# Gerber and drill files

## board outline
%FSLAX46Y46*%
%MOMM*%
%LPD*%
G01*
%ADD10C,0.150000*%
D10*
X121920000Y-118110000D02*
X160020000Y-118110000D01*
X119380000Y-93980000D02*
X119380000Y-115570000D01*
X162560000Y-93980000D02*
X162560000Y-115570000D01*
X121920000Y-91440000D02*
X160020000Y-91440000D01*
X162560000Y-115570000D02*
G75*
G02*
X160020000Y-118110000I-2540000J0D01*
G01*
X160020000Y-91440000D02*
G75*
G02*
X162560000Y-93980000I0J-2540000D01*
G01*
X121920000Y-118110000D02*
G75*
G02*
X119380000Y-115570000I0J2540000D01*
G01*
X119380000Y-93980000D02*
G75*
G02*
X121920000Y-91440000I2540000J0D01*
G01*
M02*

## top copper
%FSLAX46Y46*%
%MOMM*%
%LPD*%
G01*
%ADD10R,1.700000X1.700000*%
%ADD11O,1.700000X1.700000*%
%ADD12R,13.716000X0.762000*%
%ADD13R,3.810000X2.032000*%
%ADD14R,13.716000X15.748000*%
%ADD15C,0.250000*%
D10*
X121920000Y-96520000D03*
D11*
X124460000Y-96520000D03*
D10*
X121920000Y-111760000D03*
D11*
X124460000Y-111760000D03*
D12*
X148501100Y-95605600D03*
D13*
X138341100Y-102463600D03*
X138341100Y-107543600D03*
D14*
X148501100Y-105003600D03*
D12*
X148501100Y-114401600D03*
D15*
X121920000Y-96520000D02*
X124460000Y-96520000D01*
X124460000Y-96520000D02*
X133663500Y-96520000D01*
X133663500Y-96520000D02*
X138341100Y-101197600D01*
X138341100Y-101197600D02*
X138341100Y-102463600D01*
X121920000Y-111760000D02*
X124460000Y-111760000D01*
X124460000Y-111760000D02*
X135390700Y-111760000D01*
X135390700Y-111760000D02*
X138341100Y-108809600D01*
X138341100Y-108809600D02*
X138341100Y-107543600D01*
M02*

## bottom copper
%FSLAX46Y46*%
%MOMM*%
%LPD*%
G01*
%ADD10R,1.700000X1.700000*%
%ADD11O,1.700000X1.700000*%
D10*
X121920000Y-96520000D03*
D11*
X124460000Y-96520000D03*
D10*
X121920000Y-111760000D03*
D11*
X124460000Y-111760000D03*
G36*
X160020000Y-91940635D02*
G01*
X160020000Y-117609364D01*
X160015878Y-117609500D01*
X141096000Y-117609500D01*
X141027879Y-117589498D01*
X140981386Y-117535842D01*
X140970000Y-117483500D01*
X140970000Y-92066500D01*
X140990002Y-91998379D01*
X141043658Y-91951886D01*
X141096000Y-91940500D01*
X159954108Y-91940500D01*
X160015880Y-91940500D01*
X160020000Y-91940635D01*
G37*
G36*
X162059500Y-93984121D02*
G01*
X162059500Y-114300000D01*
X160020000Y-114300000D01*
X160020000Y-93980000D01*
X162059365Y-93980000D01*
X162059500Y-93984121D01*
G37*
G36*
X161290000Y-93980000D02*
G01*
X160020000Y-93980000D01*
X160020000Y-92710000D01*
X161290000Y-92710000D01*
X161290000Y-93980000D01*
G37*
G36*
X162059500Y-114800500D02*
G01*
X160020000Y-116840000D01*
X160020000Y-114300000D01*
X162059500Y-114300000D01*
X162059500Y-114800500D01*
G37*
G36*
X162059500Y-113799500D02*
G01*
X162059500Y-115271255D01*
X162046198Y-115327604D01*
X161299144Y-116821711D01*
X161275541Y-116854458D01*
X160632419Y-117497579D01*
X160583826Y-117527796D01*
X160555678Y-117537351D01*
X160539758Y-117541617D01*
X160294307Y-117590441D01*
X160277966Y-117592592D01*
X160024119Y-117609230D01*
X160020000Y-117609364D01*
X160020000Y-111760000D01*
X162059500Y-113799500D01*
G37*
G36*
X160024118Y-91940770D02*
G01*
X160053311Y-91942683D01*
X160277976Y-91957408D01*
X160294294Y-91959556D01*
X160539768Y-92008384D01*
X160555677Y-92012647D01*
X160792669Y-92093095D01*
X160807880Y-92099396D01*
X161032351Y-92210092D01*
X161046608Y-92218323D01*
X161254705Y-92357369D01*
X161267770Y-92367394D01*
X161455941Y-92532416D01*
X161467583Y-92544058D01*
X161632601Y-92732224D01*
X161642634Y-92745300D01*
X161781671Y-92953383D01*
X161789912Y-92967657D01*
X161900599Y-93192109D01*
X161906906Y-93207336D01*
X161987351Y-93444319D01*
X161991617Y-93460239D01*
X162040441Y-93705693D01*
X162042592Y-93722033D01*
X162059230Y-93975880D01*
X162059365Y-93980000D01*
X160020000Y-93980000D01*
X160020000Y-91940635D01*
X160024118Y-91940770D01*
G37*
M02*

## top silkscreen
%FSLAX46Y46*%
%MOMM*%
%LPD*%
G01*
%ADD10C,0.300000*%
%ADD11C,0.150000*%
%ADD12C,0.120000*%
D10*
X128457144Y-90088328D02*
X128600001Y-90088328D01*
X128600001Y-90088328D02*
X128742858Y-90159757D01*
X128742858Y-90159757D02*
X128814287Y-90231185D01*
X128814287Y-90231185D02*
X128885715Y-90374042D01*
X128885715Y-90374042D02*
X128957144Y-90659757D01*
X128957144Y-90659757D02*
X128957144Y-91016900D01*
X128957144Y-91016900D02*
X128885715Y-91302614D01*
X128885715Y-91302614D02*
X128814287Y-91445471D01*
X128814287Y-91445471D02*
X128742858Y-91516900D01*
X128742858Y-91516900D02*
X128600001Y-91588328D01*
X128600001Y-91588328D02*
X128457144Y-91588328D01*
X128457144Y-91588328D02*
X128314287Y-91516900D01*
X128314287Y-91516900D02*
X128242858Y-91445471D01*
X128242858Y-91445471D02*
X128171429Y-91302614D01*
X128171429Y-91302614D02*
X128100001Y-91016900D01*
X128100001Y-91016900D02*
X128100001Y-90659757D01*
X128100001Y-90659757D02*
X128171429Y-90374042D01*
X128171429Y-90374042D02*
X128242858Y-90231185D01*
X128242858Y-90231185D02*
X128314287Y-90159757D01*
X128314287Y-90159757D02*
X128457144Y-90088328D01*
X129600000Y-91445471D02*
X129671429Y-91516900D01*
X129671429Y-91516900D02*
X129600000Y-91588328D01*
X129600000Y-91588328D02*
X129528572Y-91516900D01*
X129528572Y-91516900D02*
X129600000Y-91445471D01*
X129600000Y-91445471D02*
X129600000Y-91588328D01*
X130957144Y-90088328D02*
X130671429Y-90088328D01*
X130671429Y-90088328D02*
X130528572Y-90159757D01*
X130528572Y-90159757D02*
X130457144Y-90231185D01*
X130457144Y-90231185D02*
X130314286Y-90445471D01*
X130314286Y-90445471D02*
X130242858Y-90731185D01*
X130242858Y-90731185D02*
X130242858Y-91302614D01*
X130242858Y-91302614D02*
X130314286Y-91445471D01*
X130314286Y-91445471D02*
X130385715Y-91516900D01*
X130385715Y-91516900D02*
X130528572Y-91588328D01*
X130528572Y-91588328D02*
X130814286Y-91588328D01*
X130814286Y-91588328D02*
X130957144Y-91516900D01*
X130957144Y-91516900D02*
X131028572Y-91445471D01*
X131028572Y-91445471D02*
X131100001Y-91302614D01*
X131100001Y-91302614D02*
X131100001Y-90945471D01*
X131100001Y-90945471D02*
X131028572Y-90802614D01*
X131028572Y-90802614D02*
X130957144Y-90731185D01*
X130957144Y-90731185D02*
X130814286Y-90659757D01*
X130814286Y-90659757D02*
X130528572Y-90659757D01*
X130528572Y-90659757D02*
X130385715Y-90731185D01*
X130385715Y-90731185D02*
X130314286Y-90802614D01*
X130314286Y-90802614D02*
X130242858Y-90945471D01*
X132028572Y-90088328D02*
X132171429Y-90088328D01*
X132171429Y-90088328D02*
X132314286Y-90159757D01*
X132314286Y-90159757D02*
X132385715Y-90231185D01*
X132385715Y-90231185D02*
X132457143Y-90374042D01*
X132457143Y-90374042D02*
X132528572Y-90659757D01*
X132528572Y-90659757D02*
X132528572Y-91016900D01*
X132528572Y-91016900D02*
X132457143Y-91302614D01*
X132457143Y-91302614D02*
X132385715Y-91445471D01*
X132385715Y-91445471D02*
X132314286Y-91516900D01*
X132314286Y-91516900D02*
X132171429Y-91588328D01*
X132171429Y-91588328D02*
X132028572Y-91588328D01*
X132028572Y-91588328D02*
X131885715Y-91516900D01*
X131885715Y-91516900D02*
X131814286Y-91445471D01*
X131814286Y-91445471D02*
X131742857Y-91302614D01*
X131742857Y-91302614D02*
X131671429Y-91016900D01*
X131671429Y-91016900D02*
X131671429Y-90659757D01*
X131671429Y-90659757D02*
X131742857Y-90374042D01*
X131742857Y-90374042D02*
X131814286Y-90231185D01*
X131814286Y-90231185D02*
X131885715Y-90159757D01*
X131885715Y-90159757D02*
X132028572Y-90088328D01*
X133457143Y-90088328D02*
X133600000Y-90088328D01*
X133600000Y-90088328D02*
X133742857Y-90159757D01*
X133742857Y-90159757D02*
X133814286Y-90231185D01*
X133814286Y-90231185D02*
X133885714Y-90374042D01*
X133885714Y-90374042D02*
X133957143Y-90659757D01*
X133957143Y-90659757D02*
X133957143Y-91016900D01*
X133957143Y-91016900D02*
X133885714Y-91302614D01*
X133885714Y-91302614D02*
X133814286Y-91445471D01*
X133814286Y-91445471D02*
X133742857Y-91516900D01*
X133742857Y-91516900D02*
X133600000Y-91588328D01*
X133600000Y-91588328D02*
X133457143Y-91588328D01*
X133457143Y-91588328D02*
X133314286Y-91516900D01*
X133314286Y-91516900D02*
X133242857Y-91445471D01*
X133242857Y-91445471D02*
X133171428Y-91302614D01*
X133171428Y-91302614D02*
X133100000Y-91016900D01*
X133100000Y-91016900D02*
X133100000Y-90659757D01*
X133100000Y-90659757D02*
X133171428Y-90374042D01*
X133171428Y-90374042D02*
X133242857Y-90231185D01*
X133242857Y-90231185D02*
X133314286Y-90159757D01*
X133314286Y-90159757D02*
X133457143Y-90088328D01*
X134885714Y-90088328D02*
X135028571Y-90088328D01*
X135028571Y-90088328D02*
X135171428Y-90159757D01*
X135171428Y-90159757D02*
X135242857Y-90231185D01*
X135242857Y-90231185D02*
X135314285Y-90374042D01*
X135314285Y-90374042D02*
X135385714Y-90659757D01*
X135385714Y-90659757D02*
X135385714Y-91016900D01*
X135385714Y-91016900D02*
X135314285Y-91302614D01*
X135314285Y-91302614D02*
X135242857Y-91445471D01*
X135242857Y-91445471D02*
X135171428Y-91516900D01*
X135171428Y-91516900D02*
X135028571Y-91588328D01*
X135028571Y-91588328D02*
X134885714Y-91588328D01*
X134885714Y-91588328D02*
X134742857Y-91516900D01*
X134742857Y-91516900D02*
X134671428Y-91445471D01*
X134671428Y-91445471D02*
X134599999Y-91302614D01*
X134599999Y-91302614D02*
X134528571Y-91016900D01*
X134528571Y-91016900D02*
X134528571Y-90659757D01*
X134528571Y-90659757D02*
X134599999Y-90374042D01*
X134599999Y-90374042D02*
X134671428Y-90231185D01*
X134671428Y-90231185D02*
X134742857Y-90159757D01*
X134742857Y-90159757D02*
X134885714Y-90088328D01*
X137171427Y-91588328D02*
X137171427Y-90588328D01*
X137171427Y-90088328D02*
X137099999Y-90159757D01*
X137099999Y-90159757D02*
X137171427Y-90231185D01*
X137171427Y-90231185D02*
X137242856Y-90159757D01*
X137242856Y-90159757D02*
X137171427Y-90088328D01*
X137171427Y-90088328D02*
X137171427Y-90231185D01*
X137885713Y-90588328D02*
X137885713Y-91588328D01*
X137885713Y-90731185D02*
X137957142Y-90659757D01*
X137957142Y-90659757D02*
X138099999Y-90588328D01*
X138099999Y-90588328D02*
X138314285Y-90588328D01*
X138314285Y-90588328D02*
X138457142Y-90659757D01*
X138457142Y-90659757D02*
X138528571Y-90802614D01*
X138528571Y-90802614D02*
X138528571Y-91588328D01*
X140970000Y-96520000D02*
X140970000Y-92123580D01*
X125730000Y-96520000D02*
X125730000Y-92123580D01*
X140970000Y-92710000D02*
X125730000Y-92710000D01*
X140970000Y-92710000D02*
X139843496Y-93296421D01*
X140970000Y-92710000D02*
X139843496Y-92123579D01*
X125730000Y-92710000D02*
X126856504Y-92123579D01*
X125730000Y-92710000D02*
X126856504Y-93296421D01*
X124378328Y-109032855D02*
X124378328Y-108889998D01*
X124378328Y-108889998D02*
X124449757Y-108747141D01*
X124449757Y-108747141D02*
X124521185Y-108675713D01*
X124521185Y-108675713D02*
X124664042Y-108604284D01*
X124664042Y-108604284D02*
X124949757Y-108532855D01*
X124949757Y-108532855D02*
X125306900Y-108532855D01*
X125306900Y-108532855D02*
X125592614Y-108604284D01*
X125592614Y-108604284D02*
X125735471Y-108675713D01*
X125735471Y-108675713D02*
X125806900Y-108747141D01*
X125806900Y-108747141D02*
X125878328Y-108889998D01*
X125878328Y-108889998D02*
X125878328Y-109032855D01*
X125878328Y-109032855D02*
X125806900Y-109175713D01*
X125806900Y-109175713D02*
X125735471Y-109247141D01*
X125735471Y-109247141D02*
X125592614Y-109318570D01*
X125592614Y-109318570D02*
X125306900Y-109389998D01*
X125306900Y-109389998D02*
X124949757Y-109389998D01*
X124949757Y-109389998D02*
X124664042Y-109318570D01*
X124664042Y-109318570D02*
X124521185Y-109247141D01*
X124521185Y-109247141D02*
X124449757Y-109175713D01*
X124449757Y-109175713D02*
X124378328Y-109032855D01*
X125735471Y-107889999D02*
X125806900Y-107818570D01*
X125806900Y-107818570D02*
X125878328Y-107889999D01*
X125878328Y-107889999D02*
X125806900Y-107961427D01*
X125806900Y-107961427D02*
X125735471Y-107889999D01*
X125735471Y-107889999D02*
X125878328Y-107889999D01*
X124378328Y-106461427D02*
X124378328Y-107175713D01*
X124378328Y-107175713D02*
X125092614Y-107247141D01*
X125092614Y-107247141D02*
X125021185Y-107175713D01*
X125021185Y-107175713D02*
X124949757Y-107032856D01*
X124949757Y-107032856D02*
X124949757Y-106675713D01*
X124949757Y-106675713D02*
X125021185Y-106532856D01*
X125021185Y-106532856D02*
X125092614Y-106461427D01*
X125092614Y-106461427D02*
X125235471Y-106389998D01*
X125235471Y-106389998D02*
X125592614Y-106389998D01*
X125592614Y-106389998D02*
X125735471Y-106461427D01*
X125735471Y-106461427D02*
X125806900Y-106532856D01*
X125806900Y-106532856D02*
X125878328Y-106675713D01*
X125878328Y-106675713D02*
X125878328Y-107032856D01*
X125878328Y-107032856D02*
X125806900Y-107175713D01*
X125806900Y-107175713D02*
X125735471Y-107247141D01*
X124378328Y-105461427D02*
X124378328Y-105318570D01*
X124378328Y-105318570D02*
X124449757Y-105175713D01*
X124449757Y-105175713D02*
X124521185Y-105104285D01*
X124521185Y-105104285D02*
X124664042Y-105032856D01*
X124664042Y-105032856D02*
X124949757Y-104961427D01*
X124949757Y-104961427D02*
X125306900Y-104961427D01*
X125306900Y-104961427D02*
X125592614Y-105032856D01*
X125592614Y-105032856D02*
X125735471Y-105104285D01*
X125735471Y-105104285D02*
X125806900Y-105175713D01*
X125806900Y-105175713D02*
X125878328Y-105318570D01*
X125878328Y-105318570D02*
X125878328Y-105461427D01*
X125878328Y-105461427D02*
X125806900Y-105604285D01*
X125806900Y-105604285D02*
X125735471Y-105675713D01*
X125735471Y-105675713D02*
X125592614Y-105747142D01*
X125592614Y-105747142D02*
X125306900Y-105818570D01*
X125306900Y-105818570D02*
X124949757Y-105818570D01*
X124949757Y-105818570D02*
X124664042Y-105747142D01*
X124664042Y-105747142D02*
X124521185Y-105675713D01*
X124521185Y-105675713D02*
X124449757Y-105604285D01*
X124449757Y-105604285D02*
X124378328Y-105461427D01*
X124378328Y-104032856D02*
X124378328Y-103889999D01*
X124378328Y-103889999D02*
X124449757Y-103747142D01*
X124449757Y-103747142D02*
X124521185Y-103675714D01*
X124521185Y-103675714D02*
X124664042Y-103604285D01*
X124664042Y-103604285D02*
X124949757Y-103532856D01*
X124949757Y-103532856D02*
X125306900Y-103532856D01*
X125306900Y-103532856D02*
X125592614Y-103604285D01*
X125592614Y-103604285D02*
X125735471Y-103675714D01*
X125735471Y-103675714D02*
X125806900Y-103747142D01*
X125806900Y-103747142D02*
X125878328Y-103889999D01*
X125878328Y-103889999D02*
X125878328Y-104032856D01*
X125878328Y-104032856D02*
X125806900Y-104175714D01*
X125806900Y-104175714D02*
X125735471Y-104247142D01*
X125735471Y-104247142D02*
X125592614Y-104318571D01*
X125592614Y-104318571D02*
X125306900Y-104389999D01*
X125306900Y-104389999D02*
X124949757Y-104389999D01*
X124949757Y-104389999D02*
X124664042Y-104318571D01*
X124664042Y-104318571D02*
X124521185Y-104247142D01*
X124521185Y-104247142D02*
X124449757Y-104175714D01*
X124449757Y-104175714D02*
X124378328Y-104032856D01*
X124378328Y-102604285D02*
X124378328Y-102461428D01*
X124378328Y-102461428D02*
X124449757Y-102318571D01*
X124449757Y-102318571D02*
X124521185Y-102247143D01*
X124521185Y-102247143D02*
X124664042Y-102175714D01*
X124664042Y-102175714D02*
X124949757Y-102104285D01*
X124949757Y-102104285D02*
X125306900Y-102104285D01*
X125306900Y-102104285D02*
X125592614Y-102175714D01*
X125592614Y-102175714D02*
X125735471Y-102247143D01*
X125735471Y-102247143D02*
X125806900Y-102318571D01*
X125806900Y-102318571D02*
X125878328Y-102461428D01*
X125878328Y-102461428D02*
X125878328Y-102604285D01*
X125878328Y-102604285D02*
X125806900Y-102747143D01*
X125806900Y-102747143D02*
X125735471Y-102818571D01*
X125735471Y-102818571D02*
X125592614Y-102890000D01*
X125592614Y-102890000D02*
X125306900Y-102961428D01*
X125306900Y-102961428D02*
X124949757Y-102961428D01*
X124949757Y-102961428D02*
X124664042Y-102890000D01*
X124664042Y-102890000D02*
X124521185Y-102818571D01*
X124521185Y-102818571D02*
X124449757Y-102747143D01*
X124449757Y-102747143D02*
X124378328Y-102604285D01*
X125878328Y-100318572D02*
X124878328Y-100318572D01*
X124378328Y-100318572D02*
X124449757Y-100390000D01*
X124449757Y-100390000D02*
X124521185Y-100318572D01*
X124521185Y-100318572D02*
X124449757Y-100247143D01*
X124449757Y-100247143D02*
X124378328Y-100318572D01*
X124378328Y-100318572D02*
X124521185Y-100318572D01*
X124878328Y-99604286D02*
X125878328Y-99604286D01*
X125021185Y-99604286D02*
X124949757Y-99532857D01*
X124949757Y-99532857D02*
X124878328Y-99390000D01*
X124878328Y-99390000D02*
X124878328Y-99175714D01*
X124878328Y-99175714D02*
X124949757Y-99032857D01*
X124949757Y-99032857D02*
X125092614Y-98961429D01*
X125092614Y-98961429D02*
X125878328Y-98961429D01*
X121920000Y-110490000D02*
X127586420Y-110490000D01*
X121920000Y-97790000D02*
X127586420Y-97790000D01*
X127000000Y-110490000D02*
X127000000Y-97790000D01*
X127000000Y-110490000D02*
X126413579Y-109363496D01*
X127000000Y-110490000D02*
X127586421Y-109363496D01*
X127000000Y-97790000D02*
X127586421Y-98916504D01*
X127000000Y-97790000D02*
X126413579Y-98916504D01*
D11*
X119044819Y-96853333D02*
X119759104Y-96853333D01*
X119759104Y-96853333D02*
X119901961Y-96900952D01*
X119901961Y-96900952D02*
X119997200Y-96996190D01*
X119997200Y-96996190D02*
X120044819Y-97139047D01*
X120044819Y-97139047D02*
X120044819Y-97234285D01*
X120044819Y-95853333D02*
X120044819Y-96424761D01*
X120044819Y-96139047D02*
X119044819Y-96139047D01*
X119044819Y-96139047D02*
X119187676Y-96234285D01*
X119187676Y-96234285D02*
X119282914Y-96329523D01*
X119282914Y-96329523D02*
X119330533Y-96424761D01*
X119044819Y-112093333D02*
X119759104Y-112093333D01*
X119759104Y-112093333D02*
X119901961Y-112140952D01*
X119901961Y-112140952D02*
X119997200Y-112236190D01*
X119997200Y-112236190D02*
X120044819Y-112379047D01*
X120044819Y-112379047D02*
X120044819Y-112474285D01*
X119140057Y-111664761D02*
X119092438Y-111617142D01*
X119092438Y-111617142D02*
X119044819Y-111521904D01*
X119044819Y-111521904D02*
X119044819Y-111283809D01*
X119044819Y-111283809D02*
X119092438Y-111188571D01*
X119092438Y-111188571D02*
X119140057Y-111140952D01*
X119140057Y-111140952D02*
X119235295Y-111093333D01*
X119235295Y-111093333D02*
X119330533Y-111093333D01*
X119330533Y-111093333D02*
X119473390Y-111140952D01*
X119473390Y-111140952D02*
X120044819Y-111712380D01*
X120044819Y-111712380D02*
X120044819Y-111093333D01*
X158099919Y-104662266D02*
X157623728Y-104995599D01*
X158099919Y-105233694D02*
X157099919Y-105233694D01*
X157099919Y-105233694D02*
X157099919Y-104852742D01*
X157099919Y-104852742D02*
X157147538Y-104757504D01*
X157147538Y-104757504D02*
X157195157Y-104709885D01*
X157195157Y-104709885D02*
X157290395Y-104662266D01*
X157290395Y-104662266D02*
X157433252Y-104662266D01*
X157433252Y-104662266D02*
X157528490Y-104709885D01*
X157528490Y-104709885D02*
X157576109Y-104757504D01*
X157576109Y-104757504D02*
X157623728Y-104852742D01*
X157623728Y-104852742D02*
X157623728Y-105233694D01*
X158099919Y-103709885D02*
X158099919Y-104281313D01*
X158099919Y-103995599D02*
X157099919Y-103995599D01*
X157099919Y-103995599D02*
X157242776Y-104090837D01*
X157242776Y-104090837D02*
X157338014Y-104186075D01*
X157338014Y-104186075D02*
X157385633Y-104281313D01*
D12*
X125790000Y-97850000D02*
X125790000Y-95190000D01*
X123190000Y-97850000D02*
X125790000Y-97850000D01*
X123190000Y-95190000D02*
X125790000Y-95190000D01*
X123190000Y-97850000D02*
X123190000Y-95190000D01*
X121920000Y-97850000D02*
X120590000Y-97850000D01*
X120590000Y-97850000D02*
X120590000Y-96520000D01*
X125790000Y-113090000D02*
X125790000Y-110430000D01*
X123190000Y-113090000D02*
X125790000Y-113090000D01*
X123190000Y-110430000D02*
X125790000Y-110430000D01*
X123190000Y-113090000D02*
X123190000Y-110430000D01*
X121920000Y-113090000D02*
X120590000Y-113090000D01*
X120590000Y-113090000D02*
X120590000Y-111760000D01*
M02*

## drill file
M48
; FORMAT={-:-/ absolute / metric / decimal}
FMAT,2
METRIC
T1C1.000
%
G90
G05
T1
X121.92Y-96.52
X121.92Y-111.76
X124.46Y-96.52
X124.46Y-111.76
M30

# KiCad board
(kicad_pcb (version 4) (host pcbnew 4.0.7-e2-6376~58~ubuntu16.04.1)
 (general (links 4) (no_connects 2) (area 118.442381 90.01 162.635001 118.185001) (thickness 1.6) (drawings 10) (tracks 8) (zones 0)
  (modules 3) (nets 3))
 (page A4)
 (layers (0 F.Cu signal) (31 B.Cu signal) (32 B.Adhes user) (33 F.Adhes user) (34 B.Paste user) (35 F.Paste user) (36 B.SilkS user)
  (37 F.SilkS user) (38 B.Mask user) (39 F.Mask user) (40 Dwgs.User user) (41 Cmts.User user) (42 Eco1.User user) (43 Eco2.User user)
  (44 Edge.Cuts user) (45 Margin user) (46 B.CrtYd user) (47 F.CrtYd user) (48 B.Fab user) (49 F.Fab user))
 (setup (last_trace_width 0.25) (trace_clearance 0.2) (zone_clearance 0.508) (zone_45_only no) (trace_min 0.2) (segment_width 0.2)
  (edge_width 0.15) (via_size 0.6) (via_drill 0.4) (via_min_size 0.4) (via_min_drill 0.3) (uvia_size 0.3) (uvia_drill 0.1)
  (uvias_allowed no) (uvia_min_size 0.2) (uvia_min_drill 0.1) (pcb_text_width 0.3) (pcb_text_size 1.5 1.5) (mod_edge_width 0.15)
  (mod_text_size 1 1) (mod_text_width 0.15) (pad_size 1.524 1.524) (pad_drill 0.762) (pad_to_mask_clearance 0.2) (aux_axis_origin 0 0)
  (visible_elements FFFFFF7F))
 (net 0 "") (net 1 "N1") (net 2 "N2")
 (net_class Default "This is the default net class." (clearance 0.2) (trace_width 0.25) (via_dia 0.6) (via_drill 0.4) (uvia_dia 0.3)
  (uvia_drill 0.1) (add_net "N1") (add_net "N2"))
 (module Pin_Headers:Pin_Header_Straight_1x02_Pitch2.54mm (layer F.Cu) (at 121.92 96.52 90)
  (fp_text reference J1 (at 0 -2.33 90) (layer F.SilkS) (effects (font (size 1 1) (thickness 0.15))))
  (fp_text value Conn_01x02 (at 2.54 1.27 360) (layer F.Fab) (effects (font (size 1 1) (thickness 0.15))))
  (fp_line (start -1.33 3.87) (end 1.33 3.87) (layer F.SilkS) (width 0.12))
  (fp_line (start -1.33 1.27) (end -1.33 3.87) (layer F.SilkS) (width 0.12))
  (fp_line (start 1.33 1.27) (end 1.33 3.87) (layer F.SilkS) (width 0.12))
  (fp_line (start -1.33 1.27) (end 1.33 1.27) (layer F.SilkS) (width 0.12))
  (fp_line (start -1.33 0) (end -1.33 -1.33) (layer F.SilkS) (width 0.12))
  (fp_line (start -1.33 -1.33) (end 0 -1.33) (layer F.SilkS) (width 0.12))
  (pad 1 thru_hole rect (at 0 0 90) (size 1.7 1.7) (drill 1) (layers *.Cu *.Mask) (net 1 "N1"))
  (pad 2 thru_hole oval (at 0 2.54 90) (size 1.7 1.7) (drill 1) (layers *.Cu *.Mask) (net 1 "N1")))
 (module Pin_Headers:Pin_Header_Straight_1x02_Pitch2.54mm (layer F.Cu) (at 121.92 111.76 90)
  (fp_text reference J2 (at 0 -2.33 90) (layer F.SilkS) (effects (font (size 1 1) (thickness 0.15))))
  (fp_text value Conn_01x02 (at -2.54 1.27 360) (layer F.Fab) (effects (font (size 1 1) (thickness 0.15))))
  (fp_line (start -1.33 3.87) (end 1.33 3.87) (layer F.SilkS) (width 0.12))
  (fp_line (start -1.33 1.27) (end -1.33 3.87) (layer F.SilkS) (width 0.12))
  (fp_line (start 1.33 1.27) (end 1.33 3.87) (layer F.SilkS) (width 0.12))
  (fp_line (start -1.33 1.27) (end 1.33 1.27) (layer F.SilkS) (width 0.12))
  (fp_line (start -1.33 0) (end -1.33 -1.33) (layer F.SilkS) (width 0.12))
  (fp_line (start -1.33 -1.33) (end 0 -1.33) (layer F.SilkS) (width 0.12))
  (pad 1 thru_hole rect (at 0 0 90) (size 1.7 1.7) (drill 1) (layers *.Cu *.Mask) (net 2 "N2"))
  (pad 2 thru_hole oval (at 0 2.54 90) (size 1.7 1.7) (drill 1) (layers *.Cu *.Mask) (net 2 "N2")))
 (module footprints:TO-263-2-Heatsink (layer F.Cu) (at 148.5011 105.0036)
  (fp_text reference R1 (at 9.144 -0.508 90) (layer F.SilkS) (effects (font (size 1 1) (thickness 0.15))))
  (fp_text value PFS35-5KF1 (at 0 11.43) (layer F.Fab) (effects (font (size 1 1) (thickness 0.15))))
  (pad "" smd rect (at 0 -9.398) (size 13.716 0.762) (layers F.Cu F.Mask))
  (pad 1 smd rect (at -10.16 -2.54) (size 3.81 2.032) (layers F.Cu F.Paste F.Mask) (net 1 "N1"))
  (pad 2 smd rect (at -10.16 2.54) (size 3.81 2.032) (layers F.Cu F.Paste F.Mask) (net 2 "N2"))
  (pad "" smd rect (at 0 0) (size 13.716 15.748) (layers F.Cu F.Paste F.Mask))
  (pad "" smd rect (at 0 9.398) (size 13.716 0.762) (layers F.Cu F.Mask)))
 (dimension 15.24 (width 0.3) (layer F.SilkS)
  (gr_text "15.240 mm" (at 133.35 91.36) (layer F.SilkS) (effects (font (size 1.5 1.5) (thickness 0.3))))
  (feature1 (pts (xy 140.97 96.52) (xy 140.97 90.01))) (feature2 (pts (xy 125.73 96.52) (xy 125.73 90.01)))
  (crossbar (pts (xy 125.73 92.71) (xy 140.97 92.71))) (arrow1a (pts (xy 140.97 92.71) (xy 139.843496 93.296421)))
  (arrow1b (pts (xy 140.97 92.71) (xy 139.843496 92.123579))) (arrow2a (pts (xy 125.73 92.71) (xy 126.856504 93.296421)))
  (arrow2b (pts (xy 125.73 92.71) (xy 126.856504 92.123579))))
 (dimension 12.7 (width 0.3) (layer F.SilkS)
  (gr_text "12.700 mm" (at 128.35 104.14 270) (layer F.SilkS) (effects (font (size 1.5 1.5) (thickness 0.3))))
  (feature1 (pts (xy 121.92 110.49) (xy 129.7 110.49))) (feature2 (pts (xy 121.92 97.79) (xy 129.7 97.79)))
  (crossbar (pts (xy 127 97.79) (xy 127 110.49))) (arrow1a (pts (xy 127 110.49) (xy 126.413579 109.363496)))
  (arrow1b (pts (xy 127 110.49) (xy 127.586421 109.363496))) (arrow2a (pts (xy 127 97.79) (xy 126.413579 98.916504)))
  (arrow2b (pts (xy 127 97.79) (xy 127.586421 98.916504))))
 (gr_line (start 121.92 118.11) (end 160.02 118.11) (angle 90) (layer Edge.Cuts) (width 0.15))
 (gr_line (start 119.38 93.98) (end 119.38 115.57) (angle 90) (layer Edge.Cuts) (width 0.15))
 (gr_line (start 162.56 93.98) (end 162.56 115.57) (angle 90) (layer Edge.Cuts) (width 0.15))
 (gr_line (start 121.92 91.44) (end 160.02 91.44) (angle 90) (layer Edge.Cuts) (width 0.15))
 (gr_arc (start 160.02 115.57) (end 162.56 115.57) (angle 90) (layer Edge.Cuts) (width 0.15))
 (gr_arc (start 160.02 93.98) (end 160.02 91.44) (angle 90) (layer Edge.Cuts) (width 0.15))
 (gr_arc (start 121.92 115.57) (end 121.92 118.11) (angle 90) (layer Edge.Cuts) (width 0.15))
 (gr_arc (start 121.92 93.98) (end 119.38 93.98) (angle 90) (layer Edge.Cuts) (width 0.15))
 (segment (start 121.92 96.52) (end 124.46 96.52) (width 0.25) (layer F.Cu) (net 1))
 (segment (start 124.46 96.52) (end 133.6635 96.52) (width 0.25) (layer F.Cu) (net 1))
 (segment (start 133.6635 96.52) (end 138.3411 101.1976) (width 0.25) (layer F.Cu) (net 1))
 (segment (start 138.3411 101.1976) (end 138.3411 102.4636) (width 0.25) (layer F.Cu) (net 1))
 (segment (start 121.92 111.76) (end 124.46 111.76) (width 0.25) (layer F.Cu) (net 2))
 (segment (start 124.46 111.76) (end 135.3907 111.76) (width 0.25) (layer F.Cu) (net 2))
 (segment (start 135.3907 111.76) (end 138.3411 108.8096) (width 0.25) (layer F.Cu) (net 2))
 (segment (start 138.3411 108.8096) (end 138.3411 107.5436) (width 0.25) (layer F.Cu) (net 2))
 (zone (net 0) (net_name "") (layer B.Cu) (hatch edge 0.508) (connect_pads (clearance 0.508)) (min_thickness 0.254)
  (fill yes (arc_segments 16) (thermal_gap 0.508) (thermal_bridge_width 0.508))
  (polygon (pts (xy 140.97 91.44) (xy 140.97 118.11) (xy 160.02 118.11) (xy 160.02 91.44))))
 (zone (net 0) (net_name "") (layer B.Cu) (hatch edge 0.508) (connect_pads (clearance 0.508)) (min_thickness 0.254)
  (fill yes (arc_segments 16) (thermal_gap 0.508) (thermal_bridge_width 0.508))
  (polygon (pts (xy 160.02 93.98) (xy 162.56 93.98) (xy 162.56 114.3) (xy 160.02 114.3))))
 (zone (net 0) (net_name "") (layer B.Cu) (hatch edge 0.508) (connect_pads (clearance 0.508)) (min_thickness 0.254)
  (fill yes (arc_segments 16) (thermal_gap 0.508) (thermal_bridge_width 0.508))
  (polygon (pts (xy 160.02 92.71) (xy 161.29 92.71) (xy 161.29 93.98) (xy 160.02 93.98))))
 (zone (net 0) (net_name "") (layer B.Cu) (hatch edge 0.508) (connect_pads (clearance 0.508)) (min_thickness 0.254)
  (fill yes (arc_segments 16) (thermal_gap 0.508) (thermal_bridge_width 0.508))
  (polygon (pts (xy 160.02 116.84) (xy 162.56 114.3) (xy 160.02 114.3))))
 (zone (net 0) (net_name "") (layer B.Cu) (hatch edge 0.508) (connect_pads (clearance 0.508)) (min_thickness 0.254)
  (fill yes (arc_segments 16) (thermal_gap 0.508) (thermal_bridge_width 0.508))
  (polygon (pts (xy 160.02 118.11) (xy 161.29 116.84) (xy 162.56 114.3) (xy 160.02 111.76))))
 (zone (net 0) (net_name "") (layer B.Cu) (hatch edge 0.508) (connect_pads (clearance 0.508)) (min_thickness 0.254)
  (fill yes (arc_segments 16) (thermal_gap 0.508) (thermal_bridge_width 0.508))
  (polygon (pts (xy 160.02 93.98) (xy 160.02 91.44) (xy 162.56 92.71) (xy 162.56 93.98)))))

